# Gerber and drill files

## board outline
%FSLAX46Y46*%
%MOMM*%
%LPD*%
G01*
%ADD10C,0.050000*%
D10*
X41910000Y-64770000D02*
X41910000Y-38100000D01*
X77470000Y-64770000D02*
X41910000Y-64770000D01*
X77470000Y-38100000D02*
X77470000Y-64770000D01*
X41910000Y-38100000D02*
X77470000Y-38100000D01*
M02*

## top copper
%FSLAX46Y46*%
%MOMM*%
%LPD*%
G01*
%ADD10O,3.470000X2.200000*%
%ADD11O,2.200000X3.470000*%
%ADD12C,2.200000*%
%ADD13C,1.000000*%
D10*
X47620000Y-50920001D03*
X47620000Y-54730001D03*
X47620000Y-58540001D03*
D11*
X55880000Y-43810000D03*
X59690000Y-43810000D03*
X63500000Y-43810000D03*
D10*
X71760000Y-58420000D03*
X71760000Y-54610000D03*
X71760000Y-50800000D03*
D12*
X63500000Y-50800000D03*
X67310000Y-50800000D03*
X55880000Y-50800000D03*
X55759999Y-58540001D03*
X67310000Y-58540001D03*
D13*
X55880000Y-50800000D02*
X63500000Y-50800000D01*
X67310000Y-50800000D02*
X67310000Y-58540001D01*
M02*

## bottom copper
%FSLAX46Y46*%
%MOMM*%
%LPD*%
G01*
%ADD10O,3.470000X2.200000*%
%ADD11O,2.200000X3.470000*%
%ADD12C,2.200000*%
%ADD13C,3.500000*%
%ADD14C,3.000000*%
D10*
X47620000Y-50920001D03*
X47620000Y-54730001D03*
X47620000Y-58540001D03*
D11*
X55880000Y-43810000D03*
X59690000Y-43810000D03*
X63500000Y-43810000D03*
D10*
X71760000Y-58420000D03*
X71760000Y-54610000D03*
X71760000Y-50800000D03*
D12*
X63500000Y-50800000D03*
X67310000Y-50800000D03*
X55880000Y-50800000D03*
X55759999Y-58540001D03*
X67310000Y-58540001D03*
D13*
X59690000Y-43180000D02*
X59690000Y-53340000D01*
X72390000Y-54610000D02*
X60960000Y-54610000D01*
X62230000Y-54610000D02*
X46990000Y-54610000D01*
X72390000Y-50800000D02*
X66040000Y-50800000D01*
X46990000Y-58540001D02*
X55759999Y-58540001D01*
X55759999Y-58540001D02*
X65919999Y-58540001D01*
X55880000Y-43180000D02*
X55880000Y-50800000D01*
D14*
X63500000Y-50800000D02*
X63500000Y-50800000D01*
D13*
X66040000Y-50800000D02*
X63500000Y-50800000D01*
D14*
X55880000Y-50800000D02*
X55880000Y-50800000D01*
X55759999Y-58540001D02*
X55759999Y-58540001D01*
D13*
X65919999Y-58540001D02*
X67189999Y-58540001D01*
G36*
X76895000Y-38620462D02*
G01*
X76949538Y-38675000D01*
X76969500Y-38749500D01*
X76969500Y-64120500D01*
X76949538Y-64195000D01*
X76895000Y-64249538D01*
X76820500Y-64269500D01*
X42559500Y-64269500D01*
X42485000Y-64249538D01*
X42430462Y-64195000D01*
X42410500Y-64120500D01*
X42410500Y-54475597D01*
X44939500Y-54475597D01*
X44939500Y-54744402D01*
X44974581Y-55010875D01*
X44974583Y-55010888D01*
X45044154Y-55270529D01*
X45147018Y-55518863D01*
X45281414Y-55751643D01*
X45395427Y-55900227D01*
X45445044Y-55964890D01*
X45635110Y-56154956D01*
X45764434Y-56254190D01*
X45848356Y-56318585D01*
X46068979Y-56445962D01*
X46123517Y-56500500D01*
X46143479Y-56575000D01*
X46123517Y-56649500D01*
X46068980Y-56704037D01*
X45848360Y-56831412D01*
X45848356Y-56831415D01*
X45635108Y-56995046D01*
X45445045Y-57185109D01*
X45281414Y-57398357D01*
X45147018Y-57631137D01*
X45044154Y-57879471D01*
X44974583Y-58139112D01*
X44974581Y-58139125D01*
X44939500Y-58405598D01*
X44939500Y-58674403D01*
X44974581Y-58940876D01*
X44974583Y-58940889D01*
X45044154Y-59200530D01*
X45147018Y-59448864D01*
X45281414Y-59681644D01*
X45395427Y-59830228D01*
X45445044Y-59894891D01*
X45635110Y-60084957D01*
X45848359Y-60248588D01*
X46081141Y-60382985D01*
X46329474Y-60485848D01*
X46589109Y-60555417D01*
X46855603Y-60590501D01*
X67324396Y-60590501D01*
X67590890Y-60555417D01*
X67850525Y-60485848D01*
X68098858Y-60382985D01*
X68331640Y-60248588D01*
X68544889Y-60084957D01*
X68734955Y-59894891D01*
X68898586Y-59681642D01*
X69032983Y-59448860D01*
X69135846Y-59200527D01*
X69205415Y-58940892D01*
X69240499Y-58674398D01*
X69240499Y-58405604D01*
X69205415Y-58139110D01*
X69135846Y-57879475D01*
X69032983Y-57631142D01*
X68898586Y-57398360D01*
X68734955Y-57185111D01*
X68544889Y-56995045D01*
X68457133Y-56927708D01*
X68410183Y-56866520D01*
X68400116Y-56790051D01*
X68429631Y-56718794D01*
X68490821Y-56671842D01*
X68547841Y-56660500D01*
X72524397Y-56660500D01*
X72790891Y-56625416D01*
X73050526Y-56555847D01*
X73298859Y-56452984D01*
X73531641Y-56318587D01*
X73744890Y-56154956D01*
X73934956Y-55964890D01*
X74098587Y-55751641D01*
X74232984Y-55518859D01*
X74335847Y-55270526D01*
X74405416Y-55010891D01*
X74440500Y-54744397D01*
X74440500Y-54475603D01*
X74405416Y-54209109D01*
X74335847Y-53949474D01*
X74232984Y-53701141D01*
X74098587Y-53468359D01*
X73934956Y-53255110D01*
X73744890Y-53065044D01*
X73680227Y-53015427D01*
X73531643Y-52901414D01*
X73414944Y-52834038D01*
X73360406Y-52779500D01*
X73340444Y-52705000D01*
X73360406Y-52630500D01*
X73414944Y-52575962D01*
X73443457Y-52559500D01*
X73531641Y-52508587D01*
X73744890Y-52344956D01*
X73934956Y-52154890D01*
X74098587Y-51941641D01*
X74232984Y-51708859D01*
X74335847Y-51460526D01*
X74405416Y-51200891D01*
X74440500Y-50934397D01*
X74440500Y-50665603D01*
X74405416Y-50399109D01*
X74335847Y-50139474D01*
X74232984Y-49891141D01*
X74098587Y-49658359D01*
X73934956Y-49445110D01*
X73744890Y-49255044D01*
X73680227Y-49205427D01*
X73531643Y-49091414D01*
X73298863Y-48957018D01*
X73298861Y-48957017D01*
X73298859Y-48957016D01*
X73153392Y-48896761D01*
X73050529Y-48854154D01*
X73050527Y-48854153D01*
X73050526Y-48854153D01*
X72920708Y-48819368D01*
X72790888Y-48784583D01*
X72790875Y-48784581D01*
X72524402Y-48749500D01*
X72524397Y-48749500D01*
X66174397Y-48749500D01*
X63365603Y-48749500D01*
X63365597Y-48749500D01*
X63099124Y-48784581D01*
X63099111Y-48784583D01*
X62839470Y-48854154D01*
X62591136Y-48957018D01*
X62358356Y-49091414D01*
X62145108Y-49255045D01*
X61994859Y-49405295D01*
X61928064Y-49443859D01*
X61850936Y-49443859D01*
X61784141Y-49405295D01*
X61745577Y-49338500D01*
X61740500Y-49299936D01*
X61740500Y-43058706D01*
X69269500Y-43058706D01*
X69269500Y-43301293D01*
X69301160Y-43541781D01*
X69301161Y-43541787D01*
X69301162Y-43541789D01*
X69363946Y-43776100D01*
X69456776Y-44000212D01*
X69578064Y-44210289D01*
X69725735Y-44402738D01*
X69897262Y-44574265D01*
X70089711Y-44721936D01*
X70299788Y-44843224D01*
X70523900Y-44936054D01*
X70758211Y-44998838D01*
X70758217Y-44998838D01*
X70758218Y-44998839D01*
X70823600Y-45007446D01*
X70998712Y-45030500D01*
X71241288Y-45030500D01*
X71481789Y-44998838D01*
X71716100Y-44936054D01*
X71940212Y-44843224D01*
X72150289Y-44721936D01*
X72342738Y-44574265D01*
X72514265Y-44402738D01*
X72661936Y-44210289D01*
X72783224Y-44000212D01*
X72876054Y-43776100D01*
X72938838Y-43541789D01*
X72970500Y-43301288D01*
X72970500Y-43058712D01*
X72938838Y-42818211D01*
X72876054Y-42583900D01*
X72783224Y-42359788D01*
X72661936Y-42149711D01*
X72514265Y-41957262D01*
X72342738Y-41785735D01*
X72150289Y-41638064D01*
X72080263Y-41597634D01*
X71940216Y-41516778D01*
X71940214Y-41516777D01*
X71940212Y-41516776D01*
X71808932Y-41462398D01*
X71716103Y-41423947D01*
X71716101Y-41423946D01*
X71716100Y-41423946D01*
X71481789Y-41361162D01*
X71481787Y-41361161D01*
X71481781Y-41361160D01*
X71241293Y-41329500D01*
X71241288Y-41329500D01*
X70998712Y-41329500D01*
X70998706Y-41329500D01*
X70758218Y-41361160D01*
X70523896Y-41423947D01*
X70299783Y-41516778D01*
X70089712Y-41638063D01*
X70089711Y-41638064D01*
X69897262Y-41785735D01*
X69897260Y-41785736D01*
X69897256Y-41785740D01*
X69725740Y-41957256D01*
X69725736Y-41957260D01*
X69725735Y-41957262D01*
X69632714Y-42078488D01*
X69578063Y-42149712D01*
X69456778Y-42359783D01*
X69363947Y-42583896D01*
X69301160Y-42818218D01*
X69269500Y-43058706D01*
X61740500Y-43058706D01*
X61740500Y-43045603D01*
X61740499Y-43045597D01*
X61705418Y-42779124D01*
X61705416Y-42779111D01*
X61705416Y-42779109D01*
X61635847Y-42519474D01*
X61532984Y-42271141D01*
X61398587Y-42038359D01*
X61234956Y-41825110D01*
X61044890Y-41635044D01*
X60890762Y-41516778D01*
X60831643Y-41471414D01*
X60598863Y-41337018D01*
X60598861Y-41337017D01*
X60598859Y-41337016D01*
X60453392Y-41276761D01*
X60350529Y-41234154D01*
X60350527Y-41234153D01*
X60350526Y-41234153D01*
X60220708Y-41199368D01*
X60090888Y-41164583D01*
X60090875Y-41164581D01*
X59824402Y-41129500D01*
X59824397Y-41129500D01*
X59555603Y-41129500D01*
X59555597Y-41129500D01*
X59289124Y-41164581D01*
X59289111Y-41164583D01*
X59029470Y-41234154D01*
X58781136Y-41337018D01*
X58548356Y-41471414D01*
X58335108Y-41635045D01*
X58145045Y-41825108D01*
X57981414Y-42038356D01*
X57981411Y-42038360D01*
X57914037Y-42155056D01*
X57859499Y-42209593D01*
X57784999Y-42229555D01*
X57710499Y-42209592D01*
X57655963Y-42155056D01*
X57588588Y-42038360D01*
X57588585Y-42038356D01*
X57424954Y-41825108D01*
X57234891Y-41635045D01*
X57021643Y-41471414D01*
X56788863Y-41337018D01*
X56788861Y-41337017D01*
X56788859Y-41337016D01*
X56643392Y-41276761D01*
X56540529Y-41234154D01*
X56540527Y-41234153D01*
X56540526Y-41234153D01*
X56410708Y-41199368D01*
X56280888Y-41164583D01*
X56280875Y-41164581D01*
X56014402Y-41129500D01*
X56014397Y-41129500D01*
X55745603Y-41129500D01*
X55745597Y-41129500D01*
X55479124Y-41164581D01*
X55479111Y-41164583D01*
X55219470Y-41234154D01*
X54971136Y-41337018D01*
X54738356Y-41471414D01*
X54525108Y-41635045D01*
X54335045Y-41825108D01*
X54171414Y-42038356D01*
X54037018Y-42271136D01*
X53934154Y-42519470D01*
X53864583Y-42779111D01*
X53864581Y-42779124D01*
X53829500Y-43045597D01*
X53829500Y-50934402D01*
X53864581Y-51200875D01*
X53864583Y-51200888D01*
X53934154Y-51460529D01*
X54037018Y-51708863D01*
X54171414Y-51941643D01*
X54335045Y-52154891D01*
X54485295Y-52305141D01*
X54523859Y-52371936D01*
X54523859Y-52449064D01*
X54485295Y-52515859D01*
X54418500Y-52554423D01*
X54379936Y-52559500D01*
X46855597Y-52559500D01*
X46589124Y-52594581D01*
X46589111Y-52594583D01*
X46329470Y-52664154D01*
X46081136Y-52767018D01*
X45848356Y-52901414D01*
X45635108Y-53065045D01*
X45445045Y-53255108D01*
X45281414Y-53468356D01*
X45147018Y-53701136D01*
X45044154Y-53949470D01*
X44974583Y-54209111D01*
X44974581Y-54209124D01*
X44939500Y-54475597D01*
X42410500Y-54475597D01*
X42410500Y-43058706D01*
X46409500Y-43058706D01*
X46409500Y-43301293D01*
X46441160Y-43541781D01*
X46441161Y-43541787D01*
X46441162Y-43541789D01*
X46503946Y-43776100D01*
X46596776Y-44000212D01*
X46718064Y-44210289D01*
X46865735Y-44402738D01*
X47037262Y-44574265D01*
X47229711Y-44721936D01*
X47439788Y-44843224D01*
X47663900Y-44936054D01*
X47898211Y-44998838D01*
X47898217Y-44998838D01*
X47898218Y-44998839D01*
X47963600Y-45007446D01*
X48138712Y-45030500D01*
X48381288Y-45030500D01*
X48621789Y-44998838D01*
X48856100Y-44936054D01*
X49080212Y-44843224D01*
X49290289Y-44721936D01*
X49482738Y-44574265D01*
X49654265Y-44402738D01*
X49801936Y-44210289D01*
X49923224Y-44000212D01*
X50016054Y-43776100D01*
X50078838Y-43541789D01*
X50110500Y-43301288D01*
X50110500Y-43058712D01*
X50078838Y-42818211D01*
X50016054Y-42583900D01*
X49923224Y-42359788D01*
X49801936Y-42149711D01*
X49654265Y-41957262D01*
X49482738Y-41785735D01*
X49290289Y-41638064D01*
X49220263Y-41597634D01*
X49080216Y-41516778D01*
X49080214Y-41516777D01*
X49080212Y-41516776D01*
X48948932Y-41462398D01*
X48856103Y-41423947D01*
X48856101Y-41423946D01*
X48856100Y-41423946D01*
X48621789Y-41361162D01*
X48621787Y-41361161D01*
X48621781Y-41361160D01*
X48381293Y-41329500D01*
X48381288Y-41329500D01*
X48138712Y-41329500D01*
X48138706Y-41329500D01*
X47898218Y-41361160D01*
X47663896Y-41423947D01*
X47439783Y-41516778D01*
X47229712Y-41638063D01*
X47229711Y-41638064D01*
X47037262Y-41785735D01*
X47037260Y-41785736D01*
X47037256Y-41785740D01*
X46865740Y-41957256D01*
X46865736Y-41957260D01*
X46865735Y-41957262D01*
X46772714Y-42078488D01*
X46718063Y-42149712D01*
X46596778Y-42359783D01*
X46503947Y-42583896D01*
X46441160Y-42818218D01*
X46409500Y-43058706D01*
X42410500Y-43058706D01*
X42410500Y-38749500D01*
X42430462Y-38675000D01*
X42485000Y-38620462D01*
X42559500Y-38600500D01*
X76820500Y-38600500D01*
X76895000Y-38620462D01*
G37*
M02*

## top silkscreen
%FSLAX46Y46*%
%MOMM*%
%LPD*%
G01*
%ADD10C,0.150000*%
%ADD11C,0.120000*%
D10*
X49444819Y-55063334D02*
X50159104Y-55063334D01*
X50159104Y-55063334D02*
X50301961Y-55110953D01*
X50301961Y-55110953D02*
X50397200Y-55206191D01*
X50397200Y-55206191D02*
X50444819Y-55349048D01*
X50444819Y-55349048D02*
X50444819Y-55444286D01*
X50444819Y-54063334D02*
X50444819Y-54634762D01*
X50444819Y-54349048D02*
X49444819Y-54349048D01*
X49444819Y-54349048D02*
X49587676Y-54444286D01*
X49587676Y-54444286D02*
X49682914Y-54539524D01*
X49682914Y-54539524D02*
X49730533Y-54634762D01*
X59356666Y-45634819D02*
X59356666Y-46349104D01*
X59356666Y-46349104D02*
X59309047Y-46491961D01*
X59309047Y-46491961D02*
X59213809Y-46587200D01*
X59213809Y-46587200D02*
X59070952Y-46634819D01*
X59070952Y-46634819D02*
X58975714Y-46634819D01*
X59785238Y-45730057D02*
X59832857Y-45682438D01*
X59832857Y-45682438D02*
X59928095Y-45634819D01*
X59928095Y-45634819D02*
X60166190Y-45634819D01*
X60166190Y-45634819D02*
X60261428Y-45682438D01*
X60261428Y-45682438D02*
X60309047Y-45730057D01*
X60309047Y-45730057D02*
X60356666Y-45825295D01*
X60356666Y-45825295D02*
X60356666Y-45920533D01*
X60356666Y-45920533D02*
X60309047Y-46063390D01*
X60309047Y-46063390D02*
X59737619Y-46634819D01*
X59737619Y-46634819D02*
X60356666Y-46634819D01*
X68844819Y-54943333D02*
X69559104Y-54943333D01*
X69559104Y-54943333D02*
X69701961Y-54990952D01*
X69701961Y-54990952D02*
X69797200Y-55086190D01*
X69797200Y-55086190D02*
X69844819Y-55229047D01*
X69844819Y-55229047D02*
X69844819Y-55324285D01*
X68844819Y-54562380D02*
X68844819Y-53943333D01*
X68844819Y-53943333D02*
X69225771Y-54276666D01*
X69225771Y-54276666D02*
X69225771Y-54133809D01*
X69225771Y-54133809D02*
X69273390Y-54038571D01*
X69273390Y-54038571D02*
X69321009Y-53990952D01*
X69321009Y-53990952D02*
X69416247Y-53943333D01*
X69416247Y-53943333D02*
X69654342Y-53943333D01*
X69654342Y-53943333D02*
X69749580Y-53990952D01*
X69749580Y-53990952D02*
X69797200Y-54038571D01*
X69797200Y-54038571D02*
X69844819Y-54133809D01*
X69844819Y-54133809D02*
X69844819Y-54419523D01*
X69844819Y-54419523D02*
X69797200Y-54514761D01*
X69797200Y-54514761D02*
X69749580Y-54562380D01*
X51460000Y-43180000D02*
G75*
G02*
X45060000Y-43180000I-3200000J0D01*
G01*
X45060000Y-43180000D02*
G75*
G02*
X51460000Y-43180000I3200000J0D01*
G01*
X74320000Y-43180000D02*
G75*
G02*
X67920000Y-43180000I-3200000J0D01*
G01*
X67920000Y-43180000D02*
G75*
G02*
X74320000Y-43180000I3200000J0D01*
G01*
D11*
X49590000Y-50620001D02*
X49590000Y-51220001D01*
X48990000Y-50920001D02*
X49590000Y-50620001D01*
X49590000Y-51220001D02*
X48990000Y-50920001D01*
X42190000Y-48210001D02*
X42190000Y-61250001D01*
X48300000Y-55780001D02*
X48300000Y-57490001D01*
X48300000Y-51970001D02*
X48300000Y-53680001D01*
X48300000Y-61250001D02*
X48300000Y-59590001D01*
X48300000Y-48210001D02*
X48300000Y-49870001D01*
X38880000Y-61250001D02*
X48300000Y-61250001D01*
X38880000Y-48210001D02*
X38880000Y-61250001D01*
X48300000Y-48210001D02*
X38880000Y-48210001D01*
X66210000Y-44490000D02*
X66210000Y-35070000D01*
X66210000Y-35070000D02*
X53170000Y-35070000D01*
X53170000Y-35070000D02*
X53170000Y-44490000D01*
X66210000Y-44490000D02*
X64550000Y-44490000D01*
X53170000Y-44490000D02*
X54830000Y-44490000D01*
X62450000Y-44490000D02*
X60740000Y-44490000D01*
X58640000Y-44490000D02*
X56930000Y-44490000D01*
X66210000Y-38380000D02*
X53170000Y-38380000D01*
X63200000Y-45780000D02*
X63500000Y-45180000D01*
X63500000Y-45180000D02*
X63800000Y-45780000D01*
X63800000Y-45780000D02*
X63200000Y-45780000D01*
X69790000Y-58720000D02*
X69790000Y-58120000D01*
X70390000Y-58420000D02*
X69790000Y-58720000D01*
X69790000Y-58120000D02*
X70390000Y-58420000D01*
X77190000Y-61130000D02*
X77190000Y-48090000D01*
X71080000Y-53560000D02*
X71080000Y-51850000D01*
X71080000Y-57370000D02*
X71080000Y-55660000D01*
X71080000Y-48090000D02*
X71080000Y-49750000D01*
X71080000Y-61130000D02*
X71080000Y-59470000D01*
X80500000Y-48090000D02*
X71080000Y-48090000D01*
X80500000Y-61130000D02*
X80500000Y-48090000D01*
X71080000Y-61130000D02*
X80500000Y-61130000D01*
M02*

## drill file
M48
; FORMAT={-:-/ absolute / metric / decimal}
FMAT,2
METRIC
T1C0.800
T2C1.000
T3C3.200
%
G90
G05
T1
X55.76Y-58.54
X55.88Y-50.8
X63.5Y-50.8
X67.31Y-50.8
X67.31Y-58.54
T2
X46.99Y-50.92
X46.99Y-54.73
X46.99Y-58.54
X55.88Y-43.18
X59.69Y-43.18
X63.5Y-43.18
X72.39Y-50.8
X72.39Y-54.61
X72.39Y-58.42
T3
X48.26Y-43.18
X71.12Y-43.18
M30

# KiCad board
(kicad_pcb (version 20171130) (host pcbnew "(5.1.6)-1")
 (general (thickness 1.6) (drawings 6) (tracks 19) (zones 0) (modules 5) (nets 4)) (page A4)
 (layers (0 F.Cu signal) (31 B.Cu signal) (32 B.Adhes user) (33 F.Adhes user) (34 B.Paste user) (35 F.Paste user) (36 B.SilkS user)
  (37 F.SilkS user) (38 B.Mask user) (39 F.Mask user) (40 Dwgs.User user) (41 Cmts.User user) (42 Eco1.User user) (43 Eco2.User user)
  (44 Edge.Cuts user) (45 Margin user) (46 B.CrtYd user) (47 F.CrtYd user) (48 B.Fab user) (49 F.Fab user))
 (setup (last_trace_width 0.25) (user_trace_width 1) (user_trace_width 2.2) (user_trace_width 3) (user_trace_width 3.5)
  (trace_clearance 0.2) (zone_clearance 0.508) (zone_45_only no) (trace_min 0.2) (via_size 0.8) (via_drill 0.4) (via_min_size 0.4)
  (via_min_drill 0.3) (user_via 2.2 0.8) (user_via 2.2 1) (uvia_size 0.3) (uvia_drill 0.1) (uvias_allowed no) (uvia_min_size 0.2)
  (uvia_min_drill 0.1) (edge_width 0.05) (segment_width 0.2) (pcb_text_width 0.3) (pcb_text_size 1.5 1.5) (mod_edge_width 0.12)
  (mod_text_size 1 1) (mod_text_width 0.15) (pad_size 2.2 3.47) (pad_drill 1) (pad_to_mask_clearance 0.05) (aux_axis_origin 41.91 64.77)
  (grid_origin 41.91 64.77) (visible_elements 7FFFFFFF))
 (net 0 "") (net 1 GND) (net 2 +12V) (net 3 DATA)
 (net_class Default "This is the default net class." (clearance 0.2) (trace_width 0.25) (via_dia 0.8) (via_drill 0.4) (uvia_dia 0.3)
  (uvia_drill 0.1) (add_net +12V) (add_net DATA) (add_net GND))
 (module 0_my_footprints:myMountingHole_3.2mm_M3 (layer F.Cu) (at 48.26 43.18)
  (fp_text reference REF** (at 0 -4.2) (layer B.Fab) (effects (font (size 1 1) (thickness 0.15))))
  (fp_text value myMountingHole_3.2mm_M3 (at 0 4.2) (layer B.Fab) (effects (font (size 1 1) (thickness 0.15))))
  (fp_circle (center 0 0) (end 3.2 0) (layer F.SilkS) (width 0.15))
  (pad "" np_thru_hole circle (at 0 0) (size 3.2 3.2) (drill 3.2) (layers *.Cu *.Mask)))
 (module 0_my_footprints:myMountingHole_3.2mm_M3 (layer F.Cu) (at 71.12 43.18)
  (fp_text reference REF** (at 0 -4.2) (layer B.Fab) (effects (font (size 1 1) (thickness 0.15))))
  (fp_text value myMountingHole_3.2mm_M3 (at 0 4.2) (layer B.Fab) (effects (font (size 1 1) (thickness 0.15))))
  (fp_circle (center 0 0) (end 3.2 0) (layer F.SilkS) (width 0.15))
  (pad "" np_thru_hole circle (at 0 0) (size 3.2 3.2) (drill 3.2) (layers *.Cu *.Mask)))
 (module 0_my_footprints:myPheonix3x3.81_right (layer F.Cu) (at 46.99 50.920001 270)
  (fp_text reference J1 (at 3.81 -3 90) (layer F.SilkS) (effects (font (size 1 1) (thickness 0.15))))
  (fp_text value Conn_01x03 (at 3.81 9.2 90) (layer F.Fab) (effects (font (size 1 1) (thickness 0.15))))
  (fp_line (start -0.3 -2.6) (end 0.3 -2.6) (layer F.SilkS) (width 0.12))
  (fp_line (start 0 -2) (end -0.3 -2.6) (layer F.SilkS) (width 0.12))
  (fp_line (start 0.3 -2.6) (end 0 -2) (layer F.SilkS) (width 0.12))
  (fp_line (start -2.71 4.8) (end 10.33 4.8) (layer F.SilkS) (width 0.12))
  (fp_line (start 4.86 -1.31) (end 6.57 -1.31) (layer F.SilkS) (width 0.12))
  (fp_line (start 1.05 -1.31) (end 2.76 -1.31) (layer F.SilkS) (width 0.12))
  (fp_line (start 10.33 -1.31) (end 8.67 -1.31) (layer F.SilkS) (width 0.12))
  (fp_line (start -2.71 -1.31) (end -1.05 -1.31) (layer F.SilkS) (width 0.12))
  (fp_line (start 10.33 8.11) (end 10.33 -1.31) (layer F.SilkS) (width 0.12))
  (fp_line (start -2.71 8.11) (end 10.33 8.11) (layer F.SilkS) (width 0.12))
  (fp_line (start -2.71 -1.31) (end -2.71 8.11) (layer F.SilkS) (width 0.12))
  (pad 1 thru_hole oval (at 0 0 270) (size 2.2 3.47) (drill 1 (offset 0 -0.63)) (layers *.Cu *.Mask) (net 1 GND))
  (pad 2 thru_hole oval (at 3.81 0 270) (size 2.2 3.47) (drill 1 (offset 0 -0.63)) (layers *.Cu *.Mask) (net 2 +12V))
  (pad 3 thru_hole oval (at 7.62 0 270) (size 2.2 3.47) (drill 1 (offset 0 -0.63)) (layers *.Cu *.Mask) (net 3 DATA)))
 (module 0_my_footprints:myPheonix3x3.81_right (layer F.Cu) (at 63.5 43.18 180)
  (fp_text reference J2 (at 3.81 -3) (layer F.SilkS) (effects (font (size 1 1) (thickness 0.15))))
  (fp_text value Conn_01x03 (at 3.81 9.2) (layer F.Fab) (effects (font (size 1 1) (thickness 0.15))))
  (fp_line (start -2.71 -1.31) (end -2.71 8.11) (layer F.SilkS) (width 0.12))
  (fp_line (start -2.71 8.11) (end 10.33 8.11) (layer F.SilkS) (width 0.12))
  (fp_line (start 10.33 8.11) (end 10.33 -1.31) (layer F.SilkS) (width 0.12))
  (fp_line (start -2.71 -1.31) (end -1.05 -1.31) (layer F.SilkS) (width 0.12))
  (fp_line (start 10.33 -1.31) (end 8.67 -1.31) (layer F.SilkS) (width 0.12))
  (fp_line (start 1.05 -1.31) (end 2.76 -1.31) (layer F.SilkS) (width 0.12))
  (fp_line (start 4.86 -1.31) (end 6.57 -1.31) (layer F.SilkS) (width 0.12))
  (fp_line (start -2.71 4.8) (end 10.33 4.8) (layer F.SilkS) (width 0.12))
  (fp_line (start 0.3 -2.6) (end 0 -2) (layer F.SilkS) (width 0.12))
  (fp_line (start 0 -2) (end -0.3 -2.6) (layer F.SilkS) (width 0.12))
  (fp_line (start -0.3 -2.6) (end 0.3 -2.6) (layer F.SilkS) (width 0.12))
  (pad 3 thru_hole oval (at 7.62 0 180) (size 2.2 3.47) (drill 1 (offset 0 -0.63)) (layers *.Cu *.Mask) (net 3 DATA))
  (pad 2 thru_hole oval (at 3.81 0 180) (size 2.2 3.47) (drill 1 (offset 0 -0.63)) (layers *.Cu *.Mask) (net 2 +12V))
  (pad 1 thru_hole oval (at 0 0 180) (size 2.2 3.47) (drill 1 (offset 0 -0.63)) (layers *.Cu *.Mask) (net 1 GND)))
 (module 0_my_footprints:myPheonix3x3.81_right (layer F.Cu) (at 72.39 58.42 90)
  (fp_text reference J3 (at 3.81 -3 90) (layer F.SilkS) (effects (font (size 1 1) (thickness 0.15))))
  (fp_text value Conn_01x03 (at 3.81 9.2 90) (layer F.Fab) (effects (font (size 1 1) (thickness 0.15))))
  (fp_line (start -0.3 -2.6) (end 0.3 -2.6) (layer F.SilkS) (width 0.12))
  (fp_line (start 0 -2) (end -0.3 -2.6) (layer F.SilkS) (width 0.12))
  (fp_line (start 0.3 -2.6) (end 0 -2) (layer F.SilkS) (width 0.12))
  (fp_line (start -2.71 4.8) (end 10.33 4.8) (layer F.SilkS) (width 0.12))
  (fp_line (start 4.86 -1.31) (end 6.57 -1.31) (layer F.SilkS) (width 0.12))
  (fp_line (start 1.05 -1.31) (end 2.76 -1.31) (layer F.SilkS) (width 0.12))
  (fp_line (start 10.33 -1.31) (end 8.67 -1.31) (layer F.SilkS) (width 0.12))
  (fp_line (start -2.71 -1.31) (end -1.05 -1.31) (layer F.SilkS) (width 0.12))
  (fp_line (start 10.33 8.11) (end 10.33 -1.31) (layer F.SilkS) (width 0.12))
  (fp_line (start -2.71 8.11) (end 10.33 8.11) (layer F.SilkS) (width 0.12))
  (fp_line (start -2.71 -1.31) (end -2.71 8.11) (layer F.SilkS) (width 0.12))
  (pad 1 thru_hole oval (at 0 0 90) (size 2.2 3.47) (drill 1 (offset 0 -0.63)) (layers *.Cu *.Mask) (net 1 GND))
  (pad 2 thru_hole oval (at 3.81 0 90) (size 2.2 3.47) (drill 1 (offset 0 -0.63)) (layers *.Cu *.Mask) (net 2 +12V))
  (pad 3 thru_hole oval (at 7.62 0 90) (size 2.2 3.47) (drill 1 (offset 0 -0.63)) (layers *.Cu *.Mask) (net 3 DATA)))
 (gr_line (start 41.91 64.77) (end 41.91 38.1) (layer Edge.Cuts) (width 0.05))
 (gr_line (start 77.47 64.77) (end 41.91 64.77) (layer Edge.Cuts) (width 0.05))
 (gr_line (start 77.47 38.1) (end 77.47 64.77) (layer Edge.Cuts) (width 0.05))
 (gr_line (start 41.91 38.1) (end 77.47 38.1) (layer Edge.Cuts) (width 0.05))
 (segment (start 59.69 43.18) (end 59.69 53.34) (width 3.5) (layer B.Cu) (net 2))
 (segment (start 72.39 54.61) (end 60.96 54.61) (width 3.5) (layer B.Cu) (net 2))
 (segment (start 62.23 54.61) (end 46.99 54.61) (width 3.5) (layer B.Cu) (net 2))
 (segment (start 72.39 50.8) (end 66.04 50.8) (width 3.5) (layer B.Cu) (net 3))
 (segment (start 46.99 58.540001) (end 55.759999 58.540001) (width 3.5) (layer B.Cu) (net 3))
 (segment (start 55.759999 58.540001) (end 65.919999 58.540001) (width 3.5) (layer B.Cu) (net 3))
 (segment (start 55.88 43.18) (end 55.88 50.8) (width 3.5) (layer B.Cu) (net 3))
 (segment (start 63.5 50.8) (end 63.5 50.8) (width 3) (layer B.Cu) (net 3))
 (via (at 63.5 50.8) (size 2.2) (drill 0.8) (layers F.Cu B.Cu) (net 3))
 (segment (start 66.04 50.8) (end 63.5 50.8) (width 3.5) (layer B.Cu) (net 3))
 (via (at 67.31 50.8) (size 2.2) (drill 0.8) (layers F.Cu B.Cu) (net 3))
 (segment (start 55.88 50.8) (end 55.88 50.8) (width 3) (layer B.Cu) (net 3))
 (via (at 55.88 50.8) (size 2.2) (drill 0.8) (layers F.Cu B.Cu) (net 3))
 (segment (start 55.759999 58.540001) (end 55.759999 58.540001) (width 3) (layer B.Cu) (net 3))
 (via (at 55.759999 58.540001) (size 2.2) (drill 0.8) (layers F.Cu B.Cu) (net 3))
 (segment (start 65.919999 58.540001) (end 67.189999 58.540001) (width 3.5) (layer B.Cu) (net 3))
 (via (at 67.31 58.540001) (size 2.2) (drill 0.8) (layers F.Cu B.Cu) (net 3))
 (segment (start 55.88 50.8) (end 63.5 50.8) (width 1) (layer F.Cu) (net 3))
 (segment (start 67.31 50.8) (end 67.31 58.540001) (width 1) (layer F.Cu) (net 3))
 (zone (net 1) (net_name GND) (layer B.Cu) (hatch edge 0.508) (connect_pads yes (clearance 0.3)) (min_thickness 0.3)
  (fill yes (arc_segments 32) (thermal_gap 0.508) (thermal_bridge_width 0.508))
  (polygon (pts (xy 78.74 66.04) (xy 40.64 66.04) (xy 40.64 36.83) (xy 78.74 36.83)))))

